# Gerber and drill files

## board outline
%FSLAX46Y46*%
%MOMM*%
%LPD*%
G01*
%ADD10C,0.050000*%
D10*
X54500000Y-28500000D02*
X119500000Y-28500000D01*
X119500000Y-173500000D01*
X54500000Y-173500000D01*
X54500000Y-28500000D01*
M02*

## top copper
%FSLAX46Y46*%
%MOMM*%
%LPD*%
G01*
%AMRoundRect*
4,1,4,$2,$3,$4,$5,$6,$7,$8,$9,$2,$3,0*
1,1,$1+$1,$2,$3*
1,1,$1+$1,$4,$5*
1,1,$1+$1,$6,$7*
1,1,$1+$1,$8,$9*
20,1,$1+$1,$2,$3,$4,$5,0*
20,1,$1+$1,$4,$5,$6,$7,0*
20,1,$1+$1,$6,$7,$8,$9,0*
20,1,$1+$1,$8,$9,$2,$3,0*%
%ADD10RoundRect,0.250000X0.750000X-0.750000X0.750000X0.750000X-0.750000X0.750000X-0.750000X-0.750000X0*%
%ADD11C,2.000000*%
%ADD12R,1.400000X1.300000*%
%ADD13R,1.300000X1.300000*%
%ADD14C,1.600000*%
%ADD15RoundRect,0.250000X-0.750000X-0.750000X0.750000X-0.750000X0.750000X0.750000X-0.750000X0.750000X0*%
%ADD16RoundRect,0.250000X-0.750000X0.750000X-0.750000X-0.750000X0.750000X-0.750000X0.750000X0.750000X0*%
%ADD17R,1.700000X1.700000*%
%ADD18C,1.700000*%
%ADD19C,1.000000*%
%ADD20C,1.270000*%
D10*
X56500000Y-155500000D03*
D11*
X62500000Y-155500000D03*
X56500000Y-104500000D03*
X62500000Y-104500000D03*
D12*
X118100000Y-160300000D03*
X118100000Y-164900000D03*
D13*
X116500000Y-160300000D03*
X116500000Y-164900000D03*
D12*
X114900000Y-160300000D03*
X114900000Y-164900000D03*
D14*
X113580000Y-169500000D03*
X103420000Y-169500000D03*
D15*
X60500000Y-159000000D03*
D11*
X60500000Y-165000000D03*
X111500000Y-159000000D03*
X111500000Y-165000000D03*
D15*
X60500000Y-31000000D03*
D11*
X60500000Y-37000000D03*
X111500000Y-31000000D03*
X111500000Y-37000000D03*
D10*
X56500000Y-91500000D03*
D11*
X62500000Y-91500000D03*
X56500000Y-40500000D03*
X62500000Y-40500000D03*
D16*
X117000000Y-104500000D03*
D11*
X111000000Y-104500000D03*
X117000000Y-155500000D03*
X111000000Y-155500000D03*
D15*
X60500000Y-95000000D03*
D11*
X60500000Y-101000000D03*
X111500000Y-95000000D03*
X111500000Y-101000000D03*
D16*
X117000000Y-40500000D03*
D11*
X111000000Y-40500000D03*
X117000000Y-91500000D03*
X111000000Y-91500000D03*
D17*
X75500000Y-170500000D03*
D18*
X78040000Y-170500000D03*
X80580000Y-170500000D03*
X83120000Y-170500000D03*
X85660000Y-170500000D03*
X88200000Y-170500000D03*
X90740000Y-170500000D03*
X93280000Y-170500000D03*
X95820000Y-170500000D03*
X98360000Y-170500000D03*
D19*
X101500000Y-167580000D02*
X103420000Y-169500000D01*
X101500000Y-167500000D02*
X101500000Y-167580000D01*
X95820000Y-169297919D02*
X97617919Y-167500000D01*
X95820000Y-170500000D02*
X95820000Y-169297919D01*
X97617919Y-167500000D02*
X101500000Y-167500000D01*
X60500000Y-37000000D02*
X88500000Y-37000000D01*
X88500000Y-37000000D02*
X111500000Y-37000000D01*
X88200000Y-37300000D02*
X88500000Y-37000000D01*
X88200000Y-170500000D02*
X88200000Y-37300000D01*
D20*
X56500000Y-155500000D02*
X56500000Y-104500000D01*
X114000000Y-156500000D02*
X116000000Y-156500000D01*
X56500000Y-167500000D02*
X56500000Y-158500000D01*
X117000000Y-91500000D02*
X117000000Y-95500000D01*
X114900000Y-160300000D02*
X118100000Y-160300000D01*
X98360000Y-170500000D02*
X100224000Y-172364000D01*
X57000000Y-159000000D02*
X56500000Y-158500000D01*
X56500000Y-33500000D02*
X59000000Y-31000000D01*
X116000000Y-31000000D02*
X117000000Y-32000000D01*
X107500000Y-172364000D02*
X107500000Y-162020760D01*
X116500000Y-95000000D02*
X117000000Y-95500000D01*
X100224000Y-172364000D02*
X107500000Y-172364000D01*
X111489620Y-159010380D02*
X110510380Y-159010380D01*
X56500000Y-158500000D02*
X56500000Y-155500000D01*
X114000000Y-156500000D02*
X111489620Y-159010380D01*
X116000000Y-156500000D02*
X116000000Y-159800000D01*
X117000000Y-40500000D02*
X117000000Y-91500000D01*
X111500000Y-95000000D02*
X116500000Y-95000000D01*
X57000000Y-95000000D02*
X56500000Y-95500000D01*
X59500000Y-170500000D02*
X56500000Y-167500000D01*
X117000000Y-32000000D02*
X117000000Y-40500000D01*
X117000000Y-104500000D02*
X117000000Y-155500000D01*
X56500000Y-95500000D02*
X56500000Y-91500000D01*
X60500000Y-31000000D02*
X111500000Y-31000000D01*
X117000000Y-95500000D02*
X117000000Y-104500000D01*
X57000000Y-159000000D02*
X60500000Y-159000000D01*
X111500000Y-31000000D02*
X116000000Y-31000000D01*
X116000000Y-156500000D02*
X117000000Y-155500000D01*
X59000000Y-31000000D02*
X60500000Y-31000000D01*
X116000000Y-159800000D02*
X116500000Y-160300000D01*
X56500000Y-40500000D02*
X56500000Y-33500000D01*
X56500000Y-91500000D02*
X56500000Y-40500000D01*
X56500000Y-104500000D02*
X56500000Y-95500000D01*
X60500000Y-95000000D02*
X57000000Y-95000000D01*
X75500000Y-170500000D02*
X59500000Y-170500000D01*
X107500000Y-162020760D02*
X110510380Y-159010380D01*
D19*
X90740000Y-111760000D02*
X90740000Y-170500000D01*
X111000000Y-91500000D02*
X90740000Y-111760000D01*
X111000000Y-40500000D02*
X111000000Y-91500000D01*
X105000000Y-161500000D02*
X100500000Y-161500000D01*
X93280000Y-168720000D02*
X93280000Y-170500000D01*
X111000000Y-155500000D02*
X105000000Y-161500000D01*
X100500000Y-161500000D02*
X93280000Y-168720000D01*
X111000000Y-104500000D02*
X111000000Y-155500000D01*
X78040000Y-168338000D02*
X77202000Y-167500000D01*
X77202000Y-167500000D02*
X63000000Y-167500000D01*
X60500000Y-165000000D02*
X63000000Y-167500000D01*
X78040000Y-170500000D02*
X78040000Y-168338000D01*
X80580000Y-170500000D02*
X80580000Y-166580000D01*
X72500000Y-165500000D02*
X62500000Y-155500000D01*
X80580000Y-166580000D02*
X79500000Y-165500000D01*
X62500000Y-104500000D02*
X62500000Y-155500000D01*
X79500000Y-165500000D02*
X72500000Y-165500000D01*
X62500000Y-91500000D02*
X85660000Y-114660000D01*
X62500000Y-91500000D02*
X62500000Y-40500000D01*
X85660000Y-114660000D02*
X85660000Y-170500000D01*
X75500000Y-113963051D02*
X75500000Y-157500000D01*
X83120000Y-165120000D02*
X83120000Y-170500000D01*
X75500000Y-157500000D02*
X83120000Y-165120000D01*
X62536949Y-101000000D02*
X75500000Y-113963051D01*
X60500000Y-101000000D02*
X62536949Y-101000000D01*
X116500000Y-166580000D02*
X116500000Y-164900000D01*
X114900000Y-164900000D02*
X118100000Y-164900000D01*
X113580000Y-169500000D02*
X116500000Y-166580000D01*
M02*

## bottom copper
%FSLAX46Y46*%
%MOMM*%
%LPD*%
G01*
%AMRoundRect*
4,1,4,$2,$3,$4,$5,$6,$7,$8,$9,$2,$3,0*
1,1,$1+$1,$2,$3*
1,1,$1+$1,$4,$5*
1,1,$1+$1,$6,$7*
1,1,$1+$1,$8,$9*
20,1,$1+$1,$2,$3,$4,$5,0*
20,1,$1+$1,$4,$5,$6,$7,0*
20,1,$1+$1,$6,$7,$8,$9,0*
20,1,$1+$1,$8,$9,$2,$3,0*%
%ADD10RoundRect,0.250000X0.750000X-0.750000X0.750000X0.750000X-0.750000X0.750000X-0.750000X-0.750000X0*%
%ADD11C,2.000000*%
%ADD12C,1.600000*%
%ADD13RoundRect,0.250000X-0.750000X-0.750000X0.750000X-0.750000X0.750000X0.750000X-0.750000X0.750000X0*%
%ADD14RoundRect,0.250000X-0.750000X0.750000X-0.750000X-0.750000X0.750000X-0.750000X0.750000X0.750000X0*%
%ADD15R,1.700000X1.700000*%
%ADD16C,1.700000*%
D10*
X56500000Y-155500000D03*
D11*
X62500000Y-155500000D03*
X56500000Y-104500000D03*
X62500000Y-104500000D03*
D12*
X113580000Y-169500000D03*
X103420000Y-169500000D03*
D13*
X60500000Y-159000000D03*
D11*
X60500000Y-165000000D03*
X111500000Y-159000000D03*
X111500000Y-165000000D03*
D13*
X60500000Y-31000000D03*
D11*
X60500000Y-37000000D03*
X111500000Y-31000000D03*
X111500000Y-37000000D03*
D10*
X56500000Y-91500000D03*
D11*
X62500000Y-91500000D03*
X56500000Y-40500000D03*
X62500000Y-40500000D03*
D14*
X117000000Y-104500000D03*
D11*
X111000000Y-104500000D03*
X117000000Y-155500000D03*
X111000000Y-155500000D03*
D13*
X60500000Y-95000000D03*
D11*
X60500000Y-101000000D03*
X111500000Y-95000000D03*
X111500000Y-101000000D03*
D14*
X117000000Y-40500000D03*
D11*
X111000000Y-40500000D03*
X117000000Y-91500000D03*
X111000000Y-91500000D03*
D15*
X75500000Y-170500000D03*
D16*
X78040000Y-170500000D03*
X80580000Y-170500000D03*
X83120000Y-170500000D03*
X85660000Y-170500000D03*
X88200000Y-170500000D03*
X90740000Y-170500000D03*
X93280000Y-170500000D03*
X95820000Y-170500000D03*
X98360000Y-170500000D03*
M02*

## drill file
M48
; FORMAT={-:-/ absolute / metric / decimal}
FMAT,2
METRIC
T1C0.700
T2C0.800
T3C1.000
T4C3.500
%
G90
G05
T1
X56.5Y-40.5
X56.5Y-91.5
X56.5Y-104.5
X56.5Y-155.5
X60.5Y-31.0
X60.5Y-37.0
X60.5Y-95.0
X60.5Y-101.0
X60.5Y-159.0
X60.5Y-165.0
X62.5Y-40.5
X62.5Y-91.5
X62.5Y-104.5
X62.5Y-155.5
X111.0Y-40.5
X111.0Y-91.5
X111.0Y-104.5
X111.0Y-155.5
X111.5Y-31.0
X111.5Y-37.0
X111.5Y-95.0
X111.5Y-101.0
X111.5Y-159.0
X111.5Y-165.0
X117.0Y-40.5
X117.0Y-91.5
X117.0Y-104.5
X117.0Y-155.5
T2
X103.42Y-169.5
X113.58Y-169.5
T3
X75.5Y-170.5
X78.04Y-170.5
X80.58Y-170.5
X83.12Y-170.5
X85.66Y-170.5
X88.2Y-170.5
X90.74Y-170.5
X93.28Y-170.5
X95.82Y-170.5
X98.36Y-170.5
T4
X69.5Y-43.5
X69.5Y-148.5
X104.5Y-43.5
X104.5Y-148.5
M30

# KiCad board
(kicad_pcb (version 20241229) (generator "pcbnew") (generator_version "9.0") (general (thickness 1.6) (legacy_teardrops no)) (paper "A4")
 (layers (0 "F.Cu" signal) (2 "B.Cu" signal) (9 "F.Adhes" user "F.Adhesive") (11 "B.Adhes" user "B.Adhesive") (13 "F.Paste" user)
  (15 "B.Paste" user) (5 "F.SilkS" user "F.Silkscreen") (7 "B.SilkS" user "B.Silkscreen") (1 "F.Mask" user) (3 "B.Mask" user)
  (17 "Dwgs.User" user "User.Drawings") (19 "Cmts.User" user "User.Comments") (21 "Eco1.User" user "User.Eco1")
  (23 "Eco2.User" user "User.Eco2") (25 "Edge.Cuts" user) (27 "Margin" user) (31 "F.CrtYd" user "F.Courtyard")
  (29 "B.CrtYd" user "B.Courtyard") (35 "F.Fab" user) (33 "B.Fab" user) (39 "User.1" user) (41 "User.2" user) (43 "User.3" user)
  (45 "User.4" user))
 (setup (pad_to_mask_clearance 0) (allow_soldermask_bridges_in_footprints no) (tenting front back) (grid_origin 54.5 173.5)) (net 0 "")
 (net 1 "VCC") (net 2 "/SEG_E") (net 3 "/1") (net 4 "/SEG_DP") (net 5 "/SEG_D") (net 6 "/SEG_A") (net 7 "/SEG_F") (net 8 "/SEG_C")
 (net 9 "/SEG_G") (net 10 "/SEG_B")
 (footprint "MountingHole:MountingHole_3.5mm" (layer "F.Cu") (at 69.5 43.5)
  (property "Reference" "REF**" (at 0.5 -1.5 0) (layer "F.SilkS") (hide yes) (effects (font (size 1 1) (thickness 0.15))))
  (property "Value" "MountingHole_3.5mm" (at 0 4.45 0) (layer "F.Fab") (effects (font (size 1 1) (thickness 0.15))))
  (pad "" np_thru_hole circle (at 0 0) (size 3.5 3.5) (drill 3.5) (layers "*.Cu" "*.Mask")))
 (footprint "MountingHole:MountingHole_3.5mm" (layer "F.Cu") (at 104.5 43.5)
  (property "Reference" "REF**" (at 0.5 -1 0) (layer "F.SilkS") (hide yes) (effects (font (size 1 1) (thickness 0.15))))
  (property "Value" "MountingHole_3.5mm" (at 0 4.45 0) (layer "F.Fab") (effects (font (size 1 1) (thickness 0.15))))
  (pad "" np_thru_hole circle (at 0 0) (size 3.5 3.5) (drill 3.5) (layers "*.Cu" "*.Mask")))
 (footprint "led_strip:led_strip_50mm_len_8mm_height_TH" (layer "F.Cu") (at 59.5 131 90)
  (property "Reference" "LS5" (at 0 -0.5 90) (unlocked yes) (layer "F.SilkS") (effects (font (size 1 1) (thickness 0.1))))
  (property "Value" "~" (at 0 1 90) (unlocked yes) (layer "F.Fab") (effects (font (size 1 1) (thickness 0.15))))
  (pad "1" thru_hole roundrect (at -24.5 -3 90) (size 2 2) (drill 0.7) (layers "*.Cu" "*.Mask") (remove_unused_layers no)
   (roundrect_rratio 0.125) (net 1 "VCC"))
  (pad "2" thru_hole circle (at -24.5 3 90) (size 2 2) (drill 0.7) (layers "*.Cu" "*.Mask") (remove_unused_layers no) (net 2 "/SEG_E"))
  (pad "3" thru_hole circle (at 26.5 -3 90) (size 2 2) (drill 0.7) (layers "*.Cu" "*.Mask") (remove_unused_layers no) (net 1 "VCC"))
  (pad "4" thru_hole circle (at 26.5 3 90) (size 2 2) (drill 0.7) (layers "*.Cu" "*.Mask") (remove_unused_layers no) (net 2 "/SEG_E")))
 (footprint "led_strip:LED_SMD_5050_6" (layer "F.Cu") (at 116.5 162.5 -90)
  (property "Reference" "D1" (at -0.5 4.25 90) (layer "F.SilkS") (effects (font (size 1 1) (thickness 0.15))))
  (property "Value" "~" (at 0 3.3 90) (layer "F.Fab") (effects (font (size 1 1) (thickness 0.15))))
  (pad "1" smd rect (at -2.2 -1.6 270) (size 1.3 1.4) (layers "F.Cu" "F.Mask" "F.Paste") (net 1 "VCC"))
  (pad "2" smd rect (at 2.4 -1.6 270) (size 1.3 1.4) (layers "F.Cu" "F.Mask" "F.Paste") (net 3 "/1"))
  (pad "3" smd rect (at -2.2 0) (size 1.3 1.3) (layers "F.Cu" "F.Mask" "F.Paste") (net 1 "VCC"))
  (pad "4" smd rect (at 2.4 0) (size 1.3 1.3) (layers "F.Cu" "F.Mask" "F.Paste") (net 3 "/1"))
  (pad "5" smd rect (at -2.2 1.6 270) (size 1.3 1.4) (layers "F.Cu" "F.Mask" "F.Paste") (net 1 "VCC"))
  (pad "6" smd rect (at 2.4 1.6 270) (size 1.3 1.4) (layers "F.Cu" "F.Mask" "F.Paste") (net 3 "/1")))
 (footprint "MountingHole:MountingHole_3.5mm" (layer "F.Cu") (at 69.5 148.5)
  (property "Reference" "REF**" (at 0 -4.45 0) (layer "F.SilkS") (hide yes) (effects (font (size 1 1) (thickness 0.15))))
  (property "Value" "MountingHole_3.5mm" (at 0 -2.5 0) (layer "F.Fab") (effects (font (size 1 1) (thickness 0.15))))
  (pad "" np_thru_hole circle (at 0 0) (size 3.5 3.5) (drill 3.5) (layers "*.Cu" "*.Mask")))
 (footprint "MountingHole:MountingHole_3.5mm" (layer "F.Cu") (at 104.5 148.5)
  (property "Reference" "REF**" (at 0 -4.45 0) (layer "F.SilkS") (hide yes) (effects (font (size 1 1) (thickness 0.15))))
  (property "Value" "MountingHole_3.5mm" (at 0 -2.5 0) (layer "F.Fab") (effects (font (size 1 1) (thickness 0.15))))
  (pad "" np_thru_hole circle (at 0 0) (size 3.5 3.5) (drill 3.5) (layers "*.Cu" "*.Mask")))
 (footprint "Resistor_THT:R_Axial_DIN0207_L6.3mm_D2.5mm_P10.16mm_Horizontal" (layer "F.Cu") (at 113.58 169.5 180)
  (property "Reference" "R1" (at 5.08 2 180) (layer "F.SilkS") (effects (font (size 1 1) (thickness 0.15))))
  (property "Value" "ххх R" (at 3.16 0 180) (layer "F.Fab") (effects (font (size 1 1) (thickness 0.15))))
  (pad "1" thru_hole circle (at 0 0 180) (size 1.6 1.6) (drill 0.8) (layers "*.Cu" "*.Mask") (remove_unused_layers no) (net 3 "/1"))
  (pad "2" thru_hole circle (at 10.16 0 180) (size 1.6 1.6) (drill 0.8) (layers "*.Cu" "*.Mask") (remove_unused_layers no) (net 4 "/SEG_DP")))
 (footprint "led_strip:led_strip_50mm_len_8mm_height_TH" (layer "F.Cu") (at 85 162)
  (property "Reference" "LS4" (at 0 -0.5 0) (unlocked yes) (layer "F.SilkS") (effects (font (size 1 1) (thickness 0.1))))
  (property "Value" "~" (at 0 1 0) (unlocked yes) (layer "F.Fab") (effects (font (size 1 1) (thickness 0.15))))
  (pad "1" thru_hole roundrect (at -24.5 -3) (size 2 2) (drill 0.7) (layers "*.Cu" "*.Mask") (remove_unused_layers no)
   (roundrect_rratio 0.125) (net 1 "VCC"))
  (pad "2" thru_hole circle (at -24.5 3) (size 2 2) (drill 0.7) (layers "*.Cu" "*.Mask") (remove_unused_layers no) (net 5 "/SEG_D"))
  (pad "3" thru_hole circle (at 26.5 -3) (size 2 2) (drill 0.7) (layers "*.Cu" "*.Mask") (remove_unused_layers no) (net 1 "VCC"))
  (pad "4" thru_hole circle (at 26.5 3) (size 2 2) (drill 0.7) (layers "*.Cu" "*.Mask") (remove_unused_layers no) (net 5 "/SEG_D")))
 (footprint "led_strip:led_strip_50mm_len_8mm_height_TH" (layer "F.Cu") (at 85 34)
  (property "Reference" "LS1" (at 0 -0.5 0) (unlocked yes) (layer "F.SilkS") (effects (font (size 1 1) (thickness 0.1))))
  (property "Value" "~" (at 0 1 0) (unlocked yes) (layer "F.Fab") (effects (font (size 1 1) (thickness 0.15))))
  (pad "1" thru_hole roundrect (at -24.5 -3) (size 2 2) (drill 0.7) (layers "*.Cu" "*.Mask") (remove_unused_layers no)
   (roundrect_rratio 0.125) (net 1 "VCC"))
  (pad "2" thru_hole circle (at -24.5 3) (size 2 2) (drill 0.7) (layers "*.Cu" "*.Mask") (remove_unused_layers no) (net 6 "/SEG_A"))
  (pad "3" thru_hole circle (at 26.5 -3) (size 2 2) (drill 0.7) (layers "*.Cu" "*.Mask") (remove_unused_layers no) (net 1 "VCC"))
  (pad "4" thru_hole circle (at 26.5 3) (size 2 2) (drill 0.7) (layers "*.Cu" "*.Mask") (remove_unused_layers no) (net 6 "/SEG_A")))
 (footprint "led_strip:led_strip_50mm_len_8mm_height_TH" (layer "F.Cu") (at 59.5 67 90)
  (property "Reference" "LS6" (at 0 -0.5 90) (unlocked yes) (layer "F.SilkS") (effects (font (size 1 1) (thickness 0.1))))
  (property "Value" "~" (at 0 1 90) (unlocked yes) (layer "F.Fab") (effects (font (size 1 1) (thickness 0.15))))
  (pad "1" thru_hole roundrect (at -24.5 -3 90) (size 2 2) (drill 0.7) (layers "*.Cu" "*.Mask") (remove_unused_layers no)
   (roundrect_rratio 0.125) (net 1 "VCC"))
  (pad "2" thru_hole circle (at -24.5 3 90) (size 2 2) (drill 0.7) (layers "*.Cu" "*.Mask") (remove_unused_layers no) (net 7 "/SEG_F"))
  (pad "3" thru_hole circle (at 26.5 -3 90) (size 2 2) (drill 0.7) (layers "*.Cu" "*.Mask") (remove_unused_layers no) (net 1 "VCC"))
  (pad "4" thru_hole circle (at 26.5 3 90) (size 2 2) (drill 0.7) (layers "*.Cu" "*.Mask") (remove_unused_layers no) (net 7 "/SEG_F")))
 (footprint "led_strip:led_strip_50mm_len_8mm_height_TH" (layer "F.Cu") (at 114 129 -90)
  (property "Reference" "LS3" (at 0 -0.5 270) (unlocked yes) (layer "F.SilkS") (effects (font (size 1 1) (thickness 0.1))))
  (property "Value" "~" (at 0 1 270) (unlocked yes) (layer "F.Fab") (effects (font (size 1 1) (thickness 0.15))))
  (pad "1" thru_hole roundrect (at -24.5 -3 270) (size 2 2) (drill 0.7) (layers "*.Cu" "*.Mask") (remove_unused_layers no)
   (roundrect_rratio 0.125) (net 1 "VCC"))
  (pad "2" thru_hole circle (at -24.5 3 270) (size 2 2) (drill 0.7) (layers "*.Cu" "*.Mask") (remove_unused_layers no) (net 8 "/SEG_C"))
  (pad "3" thru_hole circle (at 26.5 -3 270) (size 2 2) (drill 0.7) (layers "*.Cu" "*.Mask") (remove_unused_layers no) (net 1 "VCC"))
  (pad "4" thru_hole circle (at 26.5 3 270) (size 2 2) (drill 0.7) (layers "*.Cu" "*.Mask") (remove_unused_layers no) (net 8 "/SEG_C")))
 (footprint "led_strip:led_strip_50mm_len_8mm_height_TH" (layer "F.Cu") (at 85 98)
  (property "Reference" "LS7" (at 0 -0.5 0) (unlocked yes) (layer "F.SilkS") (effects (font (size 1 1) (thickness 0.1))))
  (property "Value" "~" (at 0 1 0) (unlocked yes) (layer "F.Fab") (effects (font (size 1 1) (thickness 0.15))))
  (pad "1" thru_hole roundrect (at -24.5 -3) (size 2 2) (drill 0.7) (layers "*.Cu" "*.Mask") (remove_unused_layers no)
   (roundrect_rratio 0.125) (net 1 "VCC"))
  (pad "2" thru_hole circle (at -24.5 3) (size 2 2) (drill 0.7) (layers "*.Cu" "*.Mask") (remove_unused_layers no) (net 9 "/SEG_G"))
  (pad "3" thru_hole circle (at 26.5 -3) (size 2 2) (drill 0.7) (layers "*.Cu" "*.Mask") (remove_unused_layers no) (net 1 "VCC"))
  (pad "4" thru_hole circle (at 26.5 3) (size 2 2) (drill 0.7) (layers "*.Cu" "*.Mask") (remove_unused_layers no) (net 9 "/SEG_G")))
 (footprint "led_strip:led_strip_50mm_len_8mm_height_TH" (layer "F.Cu") (at 114 65 -90)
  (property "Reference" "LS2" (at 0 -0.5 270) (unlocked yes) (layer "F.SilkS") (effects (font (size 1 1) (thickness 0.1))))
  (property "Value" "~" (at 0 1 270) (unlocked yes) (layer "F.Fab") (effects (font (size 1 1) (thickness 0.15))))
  (pad "1" thru_hole roundrect (at -24.5 -3 270) (size 2 2) (drill 0.7) (layers "*.Cu" "*.Mask") (remove_unused_layers no)
   (roundrect_rratio 0.125) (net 1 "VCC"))
  (pad "2" thru_hole circle (at -24.5 3 270) (size 2 2) (drill 0.7) (layers "*.Cu" "*.Mask") (remove_unused_layers no) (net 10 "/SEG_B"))
  (pad "3" thru_hole circle (at 26.5 -3 270) (size 2 2) (drill 0.7) (layers "*.Cu" "*.Mask") (remove_unused_layers no) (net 1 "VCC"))
  (pad "4" thru_hole circle (at 26.5 3 270) (size 2 2) (drill 0.7) (layers "*.Cu" "*.Mask") (remove_unused_layers no) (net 10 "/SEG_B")))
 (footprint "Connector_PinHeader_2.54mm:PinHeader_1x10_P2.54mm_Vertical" (layer "F.Cu") (at 75.5 170.5 90)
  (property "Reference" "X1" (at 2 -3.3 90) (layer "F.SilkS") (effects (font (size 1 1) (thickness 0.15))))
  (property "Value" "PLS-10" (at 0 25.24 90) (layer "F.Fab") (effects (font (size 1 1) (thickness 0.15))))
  (pad "1" thru_hole rect (at 0 0 90) (size 1.7 1.7) (drill 1) (layers "*.Cu" "*.Mask") (remove_unused_layers no) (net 1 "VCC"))
  (pad "2" thru_hole circle (at 0 2.54 90) (size 1.7 1.7) (drill 1) (layers "*.Cu" "*.Mask") (remove_unused_layers no) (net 5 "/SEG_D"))
  (pad "3" thru_hole circle (at 0 5.08 90) (size 1.7 1.7) (drill 1) (layers "*.Cu" "*.Mask") (remove_unused_layers no) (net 2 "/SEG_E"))
  (pad "4" thru_hole circle (at 0 7.62 90) (size 1.7 1.7) (drill 1) (layers "*.Cu" "*.Mask") (remove_unused_layers no) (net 9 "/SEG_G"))
  (pad "5" thru_hole circle (at 0 10.16 90) (size 1.7 1.7) (drill 1) (layers "*.Cu" "*.Mask") (remove_unused_layers no) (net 7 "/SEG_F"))
  (pad "6" thru_hole circle (at 0 12.7 90) (size 1.7 1.7) (drill 1) (layers "*.Cu" "*.Mask") (remove_unused_layers no) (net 6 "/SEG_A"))
  (pad "7" thru_hole circle (at 0 15.24 90) (size 1.7 1.7) (drill 1) (layers "*.Cu" "*.Mask") (remove_unused_layers no) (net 10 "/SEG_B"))
  (pad "8" thru_hole circle (at 0 17.78 90) (size 1.7 1.7) (drill 1) (layers "*.Cu" "*.Mask") (remove_unused_layers no) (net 8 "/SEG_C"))
  (pad "9" thru_hole circle (at 0 20.32 90) (size 1.7 1.7) (drill 1) (layers "*.Cu" "*.Mask") (remove_unused_layers no) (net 4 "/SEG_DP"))
  (pad "10" thru_hole circle (at 0 22.86 90) (size 1.7 1.7) (drill 1) (layers "*.Cu" "*.Mask") (remove_unused_layers no) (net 1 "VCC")))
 (gr_rect (start 54.5 28.5) (end 119.5 173.5) (stroke (width 0.05) (type default)) (fill no) (layer "Edge.Cuts"))
 (segment (start 101.5 167.58) (end 103.42 169.5) (width 1) (layer "F.Cu") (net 4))
 (segment (start 101.5 167.5) (end 101.5 167.58) (width 1) (layer "F.Cu") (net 4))
 (segment (start 95.82 169.297919) (end 97.617919 167.5) (width 1) (layer "F.Cu") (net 4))
 (segment (start 95.82 170.5) (end 95.82 169.297919) (width 1) (layer "F.Cu") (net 4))
 (segment (start 97.617919 167.5) (end 101.5 167.5) (width 1) (layer "F.Cu") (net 4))
 (segment (start 60.5 37) (end 88.5 37) (width 1) (layer "F.Cu") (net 6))
 (segment (start 88.5 37) (end 111.5 37) (width 1) (layer "F.Cu") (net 6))
 (segment (start 88.2 37.3) (end 88.5 37) (width 1) (layer "F.Cu") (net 6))
 (segment (start 88.2 170.5) (end 88.2 37.3) (width 1) (layer "F.Cu") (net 6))
 (segment (start 56.5 155.5) (end 56.5 104.5) (width 1.27) (layer "F.Cu") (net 1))
 (segment (start 114 156.5) (end 116 156.5) (width 1.27) (layer "F.Cu") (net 1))
 (segment (start 56.5 167.5) (end 56.5 158.5) (width 1.27) (layer "F.Cu") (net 1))
 (segment (start 117 91.5) (end 117 95.5) (width 1.27) (layer "F.Cu") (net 1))
 (segment (start 114.9 160.3) (end 118.1 160.3) (width 1.27) (layer "F.Cu") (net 1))
 (segment (start 98.36 170.5) (end 100.224 172.364) (width 1.27) (layer "F.Cu") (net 1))
 (segment (start 57 159) (end 56.5 158.5) (width 1.27) (layer "F.Cu") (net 1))
 (segment (start 56.5 33.5) (end 59 31) (width 1.27) (layer "F.Cu") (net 1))
 (segment (start 116 31) (end 117 32) (width 1.27) (layer "F.Cu") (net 1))
 (segment (start 107.5 172.364) (end 107.5 162.02076) (width 1.27) (layer "F.Cu") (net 1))
 (segment (start 116.5 95) (end 117 95.5) (width 1.27) (layer "F.Cu") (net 1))
 (segment (start 100.224 172.364) (end 107.5 172.364) (width 1.27) (layer "F.Cu") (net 1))
 (segment (start 111.48962 159.01038) (end 110.51038 159.01038) (width 1.27) (layer "F.Cu") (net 1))
 (segment (start 56.5 158.5) (end 56.5 155.5) (width 1.27) (layer "F.Cu") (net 1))
 (segment (start 114 156.5) (end 111.48962 159.01038) (width 1.27) (layer "F.Cu") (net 1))
 (segment (start 116 156.5) (end 116 159.8) (width 1.27) (layer "F.Cu") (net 1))
 (segment (start 117 40.5) (end 117 91.5) (width 1.27) (layer "F.Cu") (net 1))
 (segment (start 111.5 95) (end 116.5 95) (width 1.27) (layer "F.Cu") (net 1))
 (segment (start 57 95) (end 56.5 95.5) (width 1.27) (layer "F.Cu") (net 1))
 (segment (start 59.5 170.5) (end 56.5 167.5) (width 1.27) (layer "F.Cu") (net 1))
 (segment (start 117 32) (end 117 40.5) (width 1.27) (layer "F.Cu") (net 1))
 (segment (start 117 104.5) (end 117 155.5) (width 1.27) (layer "F.Cu") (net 1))
 (segment (start 56.5 95.5) (end 56.5 91.5) (width 1.27) (layer "F.Cu") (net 1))
 (segment (start 60.5 31) (end 111.5 31) (width 1.27) (layer "F.Cu") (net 1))
 (segment (start 117 95.5) (end 117 104.5) (width 1.27) (layer "F.Cu") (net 1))
 (segment (start 57 159) (end 60.5 159) (width 1.27) (layer "F.Cu") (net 1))
 (segment (start 111.5 31) (end 116 31) (width 1.27) (layer "F.Cu") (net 1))
 (segment (start 116 156.5) (end 117 155.5) (width 1.27) (layer "F.Cu") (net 1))
 (segment (start 59 31) (end 60.5 31) (width 1.27) (layer "F.Cu") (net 1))
 (segment (start 116 159.8) (end 116.5 160.3) (width 1.27) (layer "F.Cu") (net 1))
 (segment (start 56.5 40.5) (end 56.5 33.5) (width 1.27) (layer "F.Cu") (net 1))
 (segment (start 56.5 91.5) (end 56.5 40.5) (width 1.27) (layer "F.Cu") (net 1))
 (segment (start 56.5 104.5) (end 56.5 95.5) (width 1.27) (layer "F.Cu") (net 1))
 (segment (start 60.5 95) (end 57 95) (width 1.27) (layer "F.Cu") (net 1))
 (segment (start 75.5 170.5) (end 59.5 170.5) (width 1.27) (layer "F.Cu") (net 1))
 (segment (start 107.5 162.02076) (end 110.51038 159.01038) (width 1.27) (layer "F.Cu") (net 1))
 (segment (start 90.74 111.76) (end 90.74 170.5) (width 1) (layer "F.Cu") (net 10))
 (segment (start 111 91.5) (end 90.74 111.76) (width 1) (layer "F.Cu") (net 10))
 (segment (start 111 40.5) (end 111 91.5) (width 1) (layer "F.Cu") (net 10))
 (segment (start 105 161.5) (end 100.5 161.5) (width 1) (layer "F.Cu") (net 8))
 (segment (start 93.28 168.72) (end 93.28 170.5) (width 1) (layer "F.Cu") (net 8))
 (segment (start 111 155.5) (end 105 161.5) (width 1) (layer "F.Cu") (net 8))
 (segment (start 100.5 161.5) (end 93.28 168.72) (width 1) (layer "F.Cu") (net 8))
 (segment (start 111 104.5) (end 111 155.5) (width 1) (layer "F.Cu") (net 8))
 (segment (start 78.04 168.338) (end 77.202 167.5) (width 1) (layer "F.Cu") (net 5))
 (segment (start 77.202 167.5) (end 63 167.5) (width 1) (layer "F.Cu") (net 5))
 (segment (start 60.5 165) (end 63 167.5) (width 1) (layer "F.Cu") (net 5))
 (segment (start 78.04 170.5) (end 78.04 168.338) (width 1) (layer "F.Cu") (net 5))
 (segment (start 80.58 170.5) (end 80.58 166.58) (width 1) (layer "F.Cu") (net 2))
 (segment (start 72.5 165.5) (end 62.5 155.5) (width 1) (layer "F.Cu") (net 2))
 (segment (start 80.58 166.58) (end 79.5 165.5) (width 1) (layer "F.Cu") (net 2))
 (segment (start 62.5 104.5) (end 62.5 155.5) (width 1) (layer "F.Cu") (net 2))
 (segment (start 79.5 165.5) (end 72.5 165.5) (width 1) (layer "F.Cu") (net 2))
 (segment (start 62.5 91.5) (end 85.66 114.66) (width 1) (layer "F.Cu") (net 7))
 (segment (start 62.5 91.5) (end 62.5 40.5) (width 1) (layer "F.Cu") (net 7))
 (segment (start 85.66 114.66) (end 85.66 170.5) (width 1) (layer "F.Cu") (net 7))
 (segment (start 75.5 113.963051) (end 75.5 157.5) (width 1) (layer "F.Cu") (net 9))
 (segment (start 83.12 165.12) (end 83.12 170.5) (width 1) (layer "F.Cu") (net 9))
 (segment (start 75.5 157.5) (end 83.12 165.12) (width 1) (layer "F.Cu") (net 9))
 (segment (start 62.536949 101) (end 75.5 113.963051) (width 1) (layer "F.Cu") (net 9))
 (segment (start 60.5 101) (end 62.536949 101) (width 1) (layer "F.Cu") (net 9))
 (segment (start 116.5 166.58) (end 116.5 164.9) (width 1) (layer "F.Cu") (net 3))
 (segment (start 114.9 164.9) (end 118.1 164.9) (width 1) (layer "F.Cu") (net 3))
 (segment (start 113.58 169.5) (end 116.5 166.58) (width 1) (layer "F.Cu") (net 3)))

